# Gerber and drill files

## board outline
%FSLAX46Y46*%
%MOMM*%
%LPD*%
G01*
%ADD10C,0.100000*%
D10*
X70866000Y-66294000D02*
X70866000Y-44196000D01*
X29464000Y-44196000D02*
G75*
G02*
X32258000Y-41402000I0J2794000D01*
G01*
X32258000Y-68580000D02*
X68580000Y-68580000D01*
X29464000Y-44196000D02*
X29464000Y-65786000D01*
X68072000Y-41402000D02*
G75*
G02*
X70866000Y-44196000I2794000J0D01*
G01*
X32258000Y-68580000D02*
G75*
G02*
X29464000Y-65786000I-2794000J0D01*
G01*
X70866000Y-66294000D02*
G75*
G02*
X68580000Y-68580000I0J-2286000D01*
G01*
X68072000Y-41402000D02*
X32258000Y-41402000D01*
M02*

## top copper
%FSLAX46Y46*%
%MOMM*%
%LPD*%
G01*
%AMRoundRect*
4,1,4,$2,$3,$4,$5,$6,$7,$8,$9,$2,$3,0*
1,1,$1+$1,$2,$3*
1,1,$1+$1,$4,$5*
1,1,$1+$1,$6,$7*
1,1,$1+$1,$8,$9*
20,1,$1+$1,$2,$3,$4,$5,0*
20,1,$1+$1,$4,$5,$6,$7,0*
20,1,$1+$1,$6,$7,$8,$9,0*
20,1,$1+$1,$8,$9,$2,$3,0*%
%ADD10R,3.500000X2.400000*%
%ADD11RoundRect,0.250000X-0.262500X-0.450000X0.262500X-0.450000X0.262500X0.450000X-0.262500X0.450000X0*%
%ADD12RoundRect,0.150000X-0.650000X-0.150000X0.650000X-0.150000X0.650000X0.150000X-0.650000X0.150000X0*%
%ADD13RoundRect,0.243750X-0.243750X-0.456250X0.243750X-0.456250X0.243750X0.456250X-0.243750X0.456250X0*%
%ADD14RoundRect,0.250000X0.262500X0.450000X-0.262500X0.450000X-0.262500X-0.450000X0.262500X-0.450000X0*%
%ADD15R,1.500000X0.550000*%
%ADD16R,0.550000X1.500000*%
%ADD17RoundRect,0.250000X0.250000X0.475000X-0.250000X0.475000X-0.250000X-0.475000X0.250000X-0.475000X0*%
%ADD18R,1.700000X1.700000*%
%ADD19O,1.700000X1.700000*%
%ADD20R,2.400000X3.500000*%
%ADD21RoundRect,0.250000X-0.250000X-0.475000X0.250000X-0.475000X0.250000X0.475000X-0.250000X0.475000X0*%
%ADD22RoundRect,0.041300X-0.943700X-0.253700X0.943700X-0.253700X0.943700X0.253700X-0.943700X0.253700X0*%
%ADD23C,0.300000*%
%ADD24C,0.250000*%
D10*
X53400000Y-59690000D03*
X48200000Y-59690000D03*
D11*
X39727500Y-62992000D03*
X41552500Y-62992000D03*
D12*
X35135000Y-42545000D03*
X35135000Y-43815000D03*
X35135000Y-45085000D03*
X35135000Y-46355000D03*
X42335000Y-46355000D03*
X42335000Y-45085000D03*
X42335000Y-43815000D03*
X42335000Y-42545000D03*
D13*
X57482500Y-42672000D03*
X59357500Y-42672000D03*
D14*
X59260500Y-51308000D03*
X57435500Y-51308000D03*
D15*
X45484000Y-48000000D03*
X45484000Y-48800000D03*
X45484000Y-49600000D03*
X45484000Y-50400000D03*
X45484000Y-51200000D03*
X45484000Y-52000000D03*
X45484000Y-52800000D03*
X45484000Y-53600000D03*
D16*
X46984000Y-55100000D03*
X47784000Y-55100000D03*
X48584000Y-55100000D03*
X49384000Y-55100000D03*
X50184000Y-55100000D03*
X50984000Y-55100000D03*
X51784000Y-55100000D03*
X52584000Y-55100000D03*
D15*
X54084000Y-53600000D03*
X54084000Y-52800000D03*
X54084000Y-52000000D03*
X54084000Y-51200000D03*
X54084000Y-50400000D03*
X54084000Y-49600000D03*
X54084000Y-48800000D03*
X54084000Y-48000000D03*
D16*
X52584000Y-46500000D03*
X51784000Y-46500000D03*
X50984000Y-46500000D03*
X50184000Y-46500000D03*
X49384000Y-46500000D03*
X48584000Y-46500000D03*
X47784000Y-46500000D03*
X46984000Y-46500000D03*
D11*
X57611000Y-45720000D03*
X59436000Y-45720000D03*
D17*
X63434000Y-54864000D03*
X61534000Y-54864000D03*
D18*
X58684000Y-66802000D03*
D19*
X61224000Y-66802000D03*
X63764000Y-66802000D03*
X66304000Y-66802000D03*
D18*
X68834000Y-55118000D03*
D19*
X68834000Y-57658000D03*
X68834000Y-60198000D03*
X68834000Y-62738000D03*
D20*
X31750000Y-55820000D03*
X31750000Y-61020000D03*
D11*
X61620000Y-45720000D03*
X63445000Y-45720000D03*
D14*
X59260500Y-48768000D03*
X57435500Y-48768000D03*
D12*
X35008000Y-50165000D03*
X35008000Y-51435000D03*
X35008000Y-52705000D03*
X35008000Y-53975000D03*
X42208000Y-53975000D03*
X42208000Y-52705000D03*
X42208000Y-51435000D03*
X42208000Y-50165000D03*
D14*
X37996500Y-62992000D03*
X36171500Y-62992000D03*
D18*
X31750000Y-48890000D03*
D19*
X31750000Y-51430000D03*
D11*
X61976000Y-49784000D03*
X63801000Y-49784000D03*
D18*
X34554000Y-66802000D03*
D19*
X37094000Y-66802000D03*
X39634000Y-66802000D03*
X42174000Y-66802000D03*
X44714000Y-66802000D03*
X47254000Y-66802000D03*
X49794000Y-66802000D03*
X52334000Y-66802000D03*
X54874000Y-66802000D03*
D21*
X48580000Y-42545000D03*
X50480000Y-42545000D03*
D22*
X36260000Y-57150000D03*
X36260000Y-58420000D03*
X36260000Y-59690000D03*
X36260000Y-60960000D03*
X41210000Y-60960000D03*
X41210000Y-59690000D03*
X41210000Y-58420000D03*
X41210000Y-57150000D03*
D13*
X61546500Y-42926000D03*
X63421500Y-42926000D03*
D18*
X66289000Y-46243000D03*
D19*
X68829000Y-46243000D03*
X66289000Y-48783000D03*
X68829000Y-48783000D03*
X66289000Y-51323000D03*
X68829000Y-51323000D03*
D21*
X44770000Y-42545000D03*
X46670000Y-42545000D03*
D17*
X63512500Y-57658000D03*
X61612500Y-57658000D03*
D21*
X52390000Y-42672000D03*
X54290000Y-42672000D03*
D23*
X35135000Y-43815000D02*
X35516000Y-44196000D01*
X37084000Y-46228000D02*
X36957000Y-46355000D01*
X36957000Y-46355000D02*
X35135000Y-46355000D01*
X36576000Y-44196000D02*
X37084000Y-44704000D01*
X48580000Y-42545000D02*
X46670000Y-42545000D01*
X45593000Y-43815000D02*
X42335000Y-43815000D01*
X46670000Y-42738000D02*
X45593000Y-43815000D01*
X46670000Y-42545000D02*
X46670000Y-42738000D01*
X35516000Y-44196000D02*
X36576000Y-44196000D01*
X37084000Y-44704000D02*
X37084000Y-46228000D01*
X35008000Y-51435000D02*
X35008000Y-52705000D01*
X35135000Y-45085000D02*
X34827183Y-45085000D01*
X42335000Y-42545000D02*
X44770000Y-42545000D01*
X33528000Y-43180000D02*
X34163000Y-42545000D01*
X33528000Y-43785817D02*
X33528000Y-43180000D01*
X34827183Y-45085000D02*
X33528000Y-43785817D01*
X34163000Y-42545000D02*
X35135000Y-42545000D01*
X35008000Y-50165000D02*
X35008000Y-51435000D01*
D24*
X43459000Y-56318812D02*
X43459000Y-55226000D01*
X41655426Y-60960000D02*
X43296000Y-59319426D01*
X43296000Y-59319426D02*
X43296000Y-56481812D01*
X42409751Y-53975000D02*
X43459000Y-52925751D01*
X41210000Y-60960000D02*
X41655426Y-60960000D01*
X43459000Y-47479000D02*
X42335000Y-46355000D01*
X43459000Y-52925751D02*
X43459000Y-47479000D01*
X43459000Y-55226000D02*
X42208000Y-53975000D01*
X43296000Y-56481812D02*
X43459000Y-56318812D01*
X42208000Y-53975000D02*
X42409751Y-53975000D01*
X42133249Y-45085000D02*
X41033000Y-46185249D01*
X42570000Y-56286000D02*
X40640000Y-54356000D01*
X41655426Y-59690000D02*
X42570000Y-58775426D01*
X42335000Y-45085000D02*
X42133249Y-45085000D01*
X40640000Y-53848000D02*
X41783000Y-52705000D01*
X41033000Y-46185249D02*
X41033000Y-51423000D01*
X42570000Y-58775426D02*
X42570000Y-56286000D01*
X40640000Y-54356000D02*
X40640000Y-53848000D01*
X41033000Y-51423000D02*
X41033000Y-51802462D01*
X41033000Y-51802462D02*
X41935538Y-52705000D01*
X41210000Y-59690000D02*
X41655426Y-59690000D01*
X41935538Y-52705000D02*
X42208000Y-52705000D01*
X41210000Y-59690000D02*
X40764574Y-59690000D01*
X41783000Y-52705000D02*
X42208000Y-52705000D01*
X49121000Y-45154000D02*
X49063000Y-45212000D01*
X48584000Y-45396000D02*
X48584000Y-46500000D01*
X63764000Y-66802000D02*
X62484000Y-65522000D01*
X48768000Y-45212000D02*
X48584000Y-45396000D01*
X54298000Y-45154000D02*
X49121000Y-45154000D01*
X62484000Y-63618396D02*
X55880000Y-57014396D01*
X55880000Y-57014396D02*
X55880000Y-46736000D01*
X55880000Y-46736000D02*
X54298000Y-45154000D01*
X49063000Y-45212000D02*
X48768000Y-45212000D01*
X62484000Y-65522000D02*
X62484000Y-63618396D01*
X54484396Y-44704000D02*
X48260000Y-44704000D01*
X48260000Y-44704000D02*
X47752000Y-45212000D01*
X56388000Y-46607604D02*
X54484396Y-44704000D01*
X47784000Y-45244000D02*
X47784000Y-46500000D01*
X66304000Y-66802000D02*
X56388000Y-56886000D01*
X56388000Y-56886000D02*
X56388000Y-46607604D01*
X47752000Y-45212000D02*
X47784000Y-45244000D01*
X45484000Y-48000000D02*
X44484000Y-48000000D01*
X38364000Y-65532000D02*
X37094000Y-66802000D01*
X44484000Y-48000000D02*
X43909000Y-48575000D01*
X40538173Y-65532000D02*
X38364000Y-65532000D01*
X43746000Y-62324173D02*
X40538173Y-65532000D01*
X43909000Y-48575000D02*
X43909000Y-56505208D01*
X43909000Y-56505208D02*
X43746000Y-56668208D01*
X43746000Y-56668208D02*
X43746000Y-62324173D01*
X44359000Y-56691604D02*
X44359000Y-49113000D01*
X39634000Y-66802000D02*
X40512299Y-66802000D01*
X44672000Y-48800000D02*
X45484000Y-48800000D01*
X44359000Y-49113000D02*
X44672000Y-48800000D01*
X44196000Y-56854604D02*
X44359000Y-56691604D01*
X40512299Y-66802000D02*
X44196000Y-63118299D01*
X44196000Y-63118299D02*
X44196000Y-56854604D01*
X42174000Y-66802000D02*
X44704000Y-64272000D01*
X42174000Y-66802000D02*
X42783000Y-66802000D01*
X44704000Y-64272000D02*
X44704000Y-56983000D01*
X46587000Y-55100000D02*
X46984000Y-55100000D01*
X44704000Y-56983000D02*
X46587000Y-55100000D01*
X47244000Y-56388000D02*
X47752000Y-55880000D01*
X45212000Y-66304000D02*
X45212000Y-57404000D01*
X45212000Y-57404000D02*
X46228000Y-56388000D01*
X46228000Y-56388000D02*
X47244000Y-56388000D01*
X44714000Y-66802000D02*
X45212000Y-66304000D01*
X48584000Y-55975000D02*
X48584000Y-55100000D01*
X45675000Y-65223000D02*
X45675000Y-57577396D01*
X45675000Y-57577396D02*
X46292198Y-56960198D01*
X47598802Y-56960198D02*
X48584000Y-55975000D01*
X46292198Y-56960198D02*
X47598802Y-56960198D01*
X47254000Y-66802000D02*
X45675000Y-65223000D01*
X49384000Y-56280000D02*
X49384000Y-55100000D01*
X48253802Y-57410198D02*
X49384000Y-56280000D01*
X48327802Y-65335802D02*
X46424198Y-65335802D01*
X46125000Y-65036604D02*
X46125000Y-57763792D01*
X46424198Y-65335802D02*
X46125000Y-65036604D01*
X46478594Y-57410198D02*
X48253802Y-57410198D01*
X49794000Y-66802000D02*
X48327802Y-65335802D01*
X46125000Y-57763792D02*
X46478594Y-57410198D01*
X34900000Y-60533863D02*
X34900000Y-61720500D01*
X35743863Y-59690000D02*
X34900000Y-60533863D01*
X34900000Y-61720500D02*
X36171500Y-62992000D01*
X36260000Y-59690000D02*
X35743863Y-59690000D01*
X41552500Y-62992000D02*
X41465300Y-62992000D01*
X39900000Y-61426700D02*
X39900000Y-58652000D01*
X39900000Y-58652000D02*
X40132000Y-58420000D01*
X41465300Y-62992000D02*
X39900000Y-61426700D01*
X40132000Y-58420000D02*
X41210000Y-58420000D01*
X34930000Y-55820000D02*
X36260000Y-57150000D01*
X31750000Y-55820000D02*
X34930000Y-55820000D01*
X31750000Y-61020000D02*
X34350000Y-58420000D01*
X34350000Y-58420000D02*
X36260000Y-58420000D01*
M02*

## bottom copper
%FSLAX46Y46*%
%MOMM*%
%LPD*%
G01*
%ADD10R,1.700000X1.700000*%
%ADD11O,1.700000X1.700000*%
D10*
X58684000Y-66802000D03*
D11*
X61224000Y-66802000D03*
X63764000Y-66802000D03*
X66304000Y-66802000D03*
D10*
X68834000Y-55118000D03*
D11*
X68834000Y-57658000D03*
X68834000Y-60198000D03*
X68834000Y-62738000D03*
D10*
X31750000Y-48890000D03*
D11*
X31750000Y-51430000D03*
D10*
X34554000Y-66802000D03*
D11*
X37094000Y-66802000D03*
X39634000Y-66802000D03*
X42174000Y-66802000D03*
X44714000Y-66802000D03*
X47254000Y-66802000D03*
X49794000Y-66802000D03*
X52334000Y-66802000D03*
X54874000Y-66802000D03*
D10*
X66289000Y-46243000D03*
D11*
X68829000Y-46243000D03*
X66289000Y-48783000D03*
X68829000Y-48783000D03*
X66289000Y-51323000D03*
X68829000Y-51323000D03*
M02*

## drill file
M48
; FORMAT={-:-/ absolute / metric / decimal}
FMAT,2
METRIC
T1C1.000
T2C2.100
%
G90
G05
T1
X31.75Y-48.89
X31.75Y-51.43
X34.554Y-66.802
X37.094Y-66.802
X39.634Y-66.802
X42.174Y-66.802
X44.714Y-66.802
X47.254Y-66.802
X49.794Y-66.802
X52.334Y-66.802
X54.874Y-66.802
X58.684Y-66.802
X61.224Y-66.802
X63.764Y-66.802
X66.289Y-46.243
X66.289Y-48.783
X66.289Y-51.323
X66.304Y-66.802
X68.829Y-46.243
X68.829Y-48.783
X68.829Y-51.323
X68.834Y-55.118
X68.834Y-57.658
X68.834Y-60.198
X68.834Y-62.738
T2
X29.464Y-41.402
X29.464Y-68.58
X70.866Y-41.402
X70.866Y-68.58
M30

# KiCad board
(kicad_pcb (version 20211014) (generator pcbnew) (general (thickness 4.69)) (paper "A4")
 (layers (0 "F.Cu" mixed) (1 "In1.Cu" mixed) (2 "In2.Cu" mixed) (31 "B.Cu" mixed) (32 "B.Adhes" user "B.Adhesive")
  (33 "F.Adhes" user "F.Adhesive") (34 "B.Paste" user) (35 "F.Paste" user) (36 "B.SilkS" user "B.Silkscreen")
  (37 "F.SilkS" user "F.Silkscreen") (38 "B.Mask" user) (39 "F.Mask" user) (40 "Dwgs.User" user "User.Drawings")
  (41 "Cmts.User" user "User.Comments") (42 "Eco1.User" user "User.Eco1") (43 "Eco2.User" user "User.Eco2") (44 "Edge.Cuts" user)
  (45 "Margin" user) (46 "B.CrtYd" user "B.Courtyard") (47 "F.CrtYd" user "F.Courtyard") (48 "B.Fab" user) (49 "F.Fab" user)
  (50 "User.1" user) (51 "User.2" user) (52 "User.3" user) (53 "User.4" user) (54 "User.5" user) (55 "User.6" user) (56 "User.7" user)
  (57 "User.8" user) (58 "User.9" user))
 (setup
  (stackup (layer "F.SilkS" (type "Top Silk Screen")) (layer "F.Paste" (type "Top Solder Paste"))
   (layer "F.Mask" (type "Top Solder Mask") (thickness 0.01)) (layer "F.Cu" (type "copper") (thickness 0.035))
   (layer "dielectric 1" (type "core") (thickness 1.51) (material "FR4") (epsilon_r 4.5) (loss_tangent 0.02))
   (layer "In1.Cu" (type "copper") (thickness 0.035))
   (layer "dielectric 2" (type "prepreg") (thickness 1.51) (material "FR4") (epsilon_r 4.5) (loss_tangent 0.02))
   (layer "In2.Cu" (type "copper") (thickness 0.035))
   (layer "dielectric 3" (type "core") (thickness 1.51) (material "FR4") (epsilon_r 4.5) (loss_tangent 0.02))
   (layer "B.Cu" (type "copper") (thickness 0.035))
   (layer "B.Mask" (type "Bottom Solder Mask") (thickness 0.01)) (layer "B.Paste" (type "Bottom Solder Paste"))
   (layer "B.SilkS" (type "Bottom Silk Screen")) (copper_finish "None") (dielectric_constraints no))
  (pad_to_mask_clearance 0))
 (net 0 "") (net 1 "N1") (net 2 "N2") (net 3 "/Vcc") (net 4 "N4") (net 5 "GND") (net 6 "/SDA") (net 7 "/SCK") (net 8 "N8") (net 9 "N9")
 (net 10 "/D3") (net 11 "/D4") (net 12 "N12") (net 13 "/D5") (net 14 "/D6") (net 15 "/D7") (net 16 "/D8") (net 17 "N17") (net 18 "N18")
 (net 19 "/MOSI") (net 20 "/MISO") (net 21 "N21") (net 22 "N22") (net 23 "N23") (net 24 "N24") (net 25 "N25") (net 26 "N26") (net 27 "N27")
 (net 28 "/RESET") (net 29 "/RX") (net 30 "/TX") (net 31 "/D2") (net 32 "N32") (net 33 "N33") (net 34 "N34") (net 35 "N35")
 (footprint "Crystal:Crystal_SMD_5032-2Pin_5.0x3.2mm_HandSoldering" (layer "F.Cu") (at 50.8 59.69 180)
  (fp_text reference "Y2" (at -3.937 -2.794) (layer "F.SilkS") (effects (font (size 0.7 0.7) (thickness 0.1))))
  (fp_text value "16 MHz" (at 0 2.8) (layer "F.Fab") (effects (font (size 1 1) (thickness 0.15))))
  (pad "1" smd rect (at -2.6 0 180) (size 3.5 2.4) (layers "F.Cu" "F.Paste" "F.Mask") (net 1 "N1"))
  (pad "2" smd rect (at 2.6 0 180) (size 3.5 2.4) (layers "F.Cu" "F.Paste" "F.Mask") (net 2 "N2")))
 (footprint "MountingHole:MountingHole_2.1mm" (layer "F.Cu") (at 29.464 68.58)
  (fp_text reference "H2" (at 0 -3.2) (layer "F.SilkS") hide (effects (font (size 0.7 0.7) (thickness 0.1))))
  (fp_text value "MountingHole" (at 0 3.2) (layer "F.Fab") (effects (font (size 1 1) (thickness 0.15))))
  (pad "" np_thru_hole circle (at 0 0) (size 2.1 2.1) (drill 2.1) (layers *.Cu *.Mask)))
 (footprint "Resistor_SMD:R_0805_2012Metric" (layer "F.Cu") (at 40.64 62.992)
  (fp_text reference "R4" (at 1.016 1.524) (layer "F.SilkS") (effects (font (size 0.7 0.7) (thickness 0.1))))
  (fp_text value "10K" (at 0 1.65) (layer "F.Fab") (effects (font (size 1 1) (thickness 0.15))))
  (pad "1" smd roundrect (at -0.9125 0) (size 1.025 1.4) (layers "F.Cu" "F.Paste" "F.Mask") (roundrect_rratio 0.243902) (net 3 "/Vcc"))
  (pad "2" smd roundrect (at 0.9125 0) (size 1.025 1.4) (layers "F.Cu" "F.Paste" "F.Mask") (roundrect_rratio 0.243902) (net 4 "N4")))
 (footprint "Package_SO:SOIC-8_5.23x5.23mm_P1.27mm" (layer "F.Cu") (at 38.735 44.45)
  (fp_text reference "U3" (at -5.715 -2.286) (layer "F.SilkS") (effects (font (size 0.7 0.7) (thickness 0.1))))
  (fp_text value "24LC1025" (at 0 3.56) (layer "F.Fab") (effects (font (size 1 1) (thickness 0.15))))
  (pad "1" smd roundrect (at -3.6 -1.905) (size 1.6 0.6) (layers "F.Cu" "F.Paste" "F.Mask") (roundrect_rratio 0.25) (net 3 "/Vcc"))
  (pad "2" smd roundrect (at -3.6 -0.635) (size 1.6 0.6) (layers "F.Cu" "F.Paste" "F.Mask") (roundrect_rratio 0.25) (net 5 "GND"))
  (pad "3" smd roundrect (at -3.6 0.635) (size 1.6 0.6) (layers "F.Cu" "F.Paste" "F.Mask") (roundrect_rratio 0.25) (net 3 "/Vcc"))
  (pad "4" smd roundrect (at -3.6 1.905) (size 1.6 0.6) (layers "F.Cu" "F.Paste" "F.Mask") (roundrect_rratio 0.25) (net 5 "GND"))
  (pad "5" smd roundrect (at 3.6 1.905) (size 1.6 0.6) (layers "F.Cu" "F.Paste" "F.Mask") (roundrect_rratio 0.25) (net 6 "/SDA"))
  (pad "6" smd roundrect (at 3.6 0.635) (size 1.6 0.6) (layers "F.Cu" "F.Paste" "F.Mask") (roundrect_rratio 0.25) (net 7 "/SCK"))
  (pad "7" smd roundrect (at 3.6 -0.635) (size 1.6 0.6) (layers "F.Cu" "F.Paste" "F.Mask") (roundrect_rratio 0.25) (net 5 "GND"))
  (pad "8" smd roundrect (at 3.6 -1.905) (size 1.6 0.6) (layers "F.Cu" "F.Paste" "F.Mask") (roundrect_rratio 0.25) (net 3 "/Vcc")))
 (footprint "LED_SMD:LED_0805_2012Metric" (layer "F.Cu") (at 58.42 42.672)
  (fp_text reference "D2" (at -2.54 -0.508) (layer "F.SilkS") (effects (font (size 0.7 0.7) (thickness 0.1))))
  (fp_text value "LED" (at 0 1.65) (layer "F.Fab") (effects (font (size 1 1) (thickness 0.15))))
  (pad "1" smd roundrect (at -0.9375 0) (size 0.975 1.4) (layers "F.Cu" "F.Paste" "F.Mask") (roundrect_rratio 0.25) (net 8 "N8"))
  (pad "2" smd roundrect (at 0.9375 0) (size 0.975 1.4) (layers "F.Cu" "F.Paste" "F.Mask") (roundrect_rratio 0.25) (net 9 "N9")))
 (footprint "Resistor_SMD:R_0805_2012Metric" (layer "F.Cu") (at 58.348 51.308 180)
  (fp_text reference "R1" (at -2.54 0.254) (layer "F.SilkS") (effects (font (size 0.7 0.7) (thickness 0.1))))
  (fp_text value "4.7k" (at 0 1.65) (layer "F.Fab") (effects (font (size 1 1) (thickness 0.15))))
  (pad "1" smd roundrect (at -0.9125 0 180) (size 1.025 1.4) (layers "F.Cu" "F.Paste" "F.Mask") (roundrect_rratio 0.243902) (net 3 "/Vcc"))
  (pad "2" smd roundrect (at 0.9125 0 180) (size 1.025 1.4) (layers "F.Cu" "F.Paste" "F.Mask") (roundrect_rratio 0.243902) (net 7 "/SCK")))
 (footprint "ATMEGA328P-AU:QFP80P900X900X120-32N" (layer "F.Cu") (at 49.784 50.8)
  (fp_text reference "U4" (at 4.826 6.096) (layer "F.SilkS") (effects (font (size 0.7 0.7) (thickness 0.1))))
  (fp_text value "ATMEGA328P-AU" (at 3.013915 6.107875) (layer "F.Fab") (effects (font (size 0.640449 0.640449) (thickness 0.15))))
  (pad "1" smd rect locked (at -4.3 -2.8) (size 1.5 0.55) (layers "F.Cu" "F.Paste" "F.Mask") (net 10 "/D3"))
  (pad "2" smd rect locked (at -4.3 -2) (size 1.5 0.55) (layers "F.Cu" "F.Paste" "F.Mask") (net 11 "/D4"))
  (pad "3" smd rect locked (at -4.3 -1.2) (size 1.5 0.55) (layers "F.Cu" "F.Paste" "F.Mask") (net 5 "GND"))
  (pad "4" smd rect locked (at -4.3 -0.4) (size 1.5 0.55) (layers "F.Cu" "F.Paste" "F.Mask") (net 9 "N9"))
  (pad "5" smd rect locked (at -4.3 0.4) (size 1.5 0.55) (layers "F.Cu" "F.Paste" "F.Mask") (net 5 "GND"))
  (pad "6" smd rect locked (at -4.3 1.2) (size 1.5 0.55) (layers "F.Cu" "F.Paste" "F.Mask") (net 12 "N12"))
  (pad "7" smd rect locked (at -4.3 2) (size 1.5 0.55) (layers "F.Cu" "F.Paste" "F.Mask") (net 2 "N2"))
  (pad "8" smd rect locked (at -4.3 2.8) (size 1.5 0.55) (layers "F.Cu" "F.Paste" "F.Mask") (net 1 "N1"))
  (pad "9" smd rect locked (at -2.8 4.3) (size 0.55 1.5) (layers "F.Cu" "F.Paste" "F.Mask") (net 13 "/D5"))
  (pad "10" smd rect locked (at -2 4.3) (size 0.55 1.5) (layers "F.Cu" "F.Paste" "F.Mask") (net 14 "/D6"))
  (pad "11" smd rect locked (at -1.2 4.3) (size 0.55 1.5) (layers "F.Cu" "F.Paste" "F.Mask") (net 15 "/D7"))
  (pad "12" smd rect locked (at -0.4 4.3) (size 0.55 1.5) (layers "F.Cu" "F.Paste" "F.Mask") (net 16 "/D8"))
  (pad "13" smd rect locked (at 0.4 4.3) (size 0.55 1.5) (layers "F.Cu" "F.Paste" "F.Mask") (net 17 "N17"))
  (pad "14" smd rect locked (at 1.2 4.3) (size 0.55 1.5) (layers "F.Cu" "F.Paste" "F.Mask") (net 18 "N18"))
  (pad "15" smd rect locked (at 2 4.3) (size 0.55 1.5) (layers "F.Cu" "F.Paste" "F.Mask") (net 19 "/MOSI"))
  (pad "16" smd rect locked (at 2.8 4.3) (size 0.55 1.5) (layers "F.Cu" "F.Paste" "F.Mask") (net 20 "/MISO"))
  (pad "17" smd rect locked (at 4.3 2.8) (size 1.5 0.55) (layers "F.Cu" "F.Paste" "F.Mask") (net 7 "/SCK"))
  (pad "18" smd rect locked (at 4.3 2) (size 1.5 0.55) (layers "F.Cu" "F.Paste" "F.Mask") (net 9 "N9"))
  (pad "19" smd rect locked (at 4.3 1.2) (size 1.5 0.55) (layers "F.Cu" "F.Paste" "F.Mask") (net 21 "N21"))
  (pad "20" smd rect locked (at 4.3 0.4) (size 1.5 0.55) (layers "F.Cu" "F.Paste" "F.Mask") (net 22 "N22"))
  (pad "21" smd rect locked (at 4.3 -0.4) (size 1.5 0.55) (layers "F.Cu" "F.Paste" "F.Mask") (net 5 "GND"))
  (pad "22" smd rect locked (at 4.3 -1.2) (size 1.5 0.55) (layers "F.Cu" "F.Paste" "F.Mask") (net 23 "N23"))
  (pad "23" smd rect locked (at 4.3 -2) (size 1.5 0.55) (layers "F.Cu" "F.Paste" "F.Mask") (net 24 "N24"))
  (pad "24" smd rect locked (at 4.3 -2.8) (size 1.5 0.55) (layers "F.Cu" "F.Paste" "F.Mask") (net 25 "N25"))
  (pad "25" smd rect locked (at 2.8 -4.3) (size 0.55 1.5) (layers "F.Cu" "F.Paste" "F.Mask") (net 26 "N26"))
  (pad "26" smd rect locked (at 2 -4.3) (size 0.55 1.5) (layers "F.Cu" "F.Paste" "F.Mask") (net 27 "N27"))
  (pad "27" smd rect locked (at 1.2 -4.3) (size 0.55 1.5) (layers "F.Cu" "F.Paste" "F.Mask") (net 6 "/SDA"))
  (pad "28" smd rect locked (at 0.4 -4.3) (size 0.55 1.5) (layers "F.Cu" "F.Paste" "F.Mask") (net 7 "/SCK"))
  (pad "29" smd rect locked (at -0.4 -4.3) (size 0.55 1.5) (layers "F.Cu" "F.Paste" "F.Mask") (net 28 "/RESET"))
  (pad "30" smd rect locked (at -1.2 -4.3) (size 0.55 1.5) (layers "F.Cu" "F.Paste" "F.Mask") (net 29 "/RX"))
  (pad "31" smd rect locked (at -2 -4.3) (size 0.55 1.5) (layers "F.Cu" "F.Paste" "F.Mask") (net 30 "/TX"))
  (pad "32" smd rect locked (at -2.8 -4.3) (size 0.55 1.5) (layers "F.Cu" "F.Paste" "F.Mask") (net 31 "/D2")))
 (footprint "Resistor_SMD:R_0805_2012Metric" (layer "F.Cu") (at 58.5235 45.72)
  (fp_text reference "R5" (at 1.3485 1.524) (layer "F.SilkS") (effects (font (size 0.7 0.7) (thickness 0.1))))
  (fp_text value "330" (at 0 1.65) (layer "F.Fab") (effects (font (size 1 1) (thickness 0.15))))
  (pad "1" smd roundrect (at -0.9125 0) (size 1.025 1.4) (layers "F.Cu" "F.Paste" "F.Mask") (roundrect_rratio 0.243902) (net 5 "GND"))
  (pad "2" smd roundrect (at 0.9125 0) (size 1.025 1.4) (layers "F.Cu" "F.Paste" "F.Mask") (roundrect_rratio 0.243902) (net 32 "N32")))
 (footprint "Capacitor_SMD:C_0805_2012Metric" (layer "F.Cu") (at 62.484 54.864 180)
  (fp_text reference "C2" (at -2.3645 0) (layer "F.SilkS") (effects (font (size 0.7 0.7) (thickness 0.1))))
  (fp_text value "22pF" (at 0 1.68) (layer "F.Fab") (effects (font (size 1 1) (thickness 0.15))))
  (pad "1" smd roundrect (at -0.95 0 180) (size 1 1.45) (layers "F.Cu" "F.Paste" "F.Mask") (roundrect_rratio 0.25) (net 5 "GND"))
  (pad "2" smd roundrect (at 0.95 0 180) (size 1 1.45) (layers "F.Cu" "F.Paste" "F.Mask") (roundrect_rratio 0.25) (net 2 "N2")))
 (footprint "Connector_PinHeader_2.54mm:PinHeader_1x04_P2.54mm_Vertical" (layer "F.Cu") (at 58.684 66.802 90)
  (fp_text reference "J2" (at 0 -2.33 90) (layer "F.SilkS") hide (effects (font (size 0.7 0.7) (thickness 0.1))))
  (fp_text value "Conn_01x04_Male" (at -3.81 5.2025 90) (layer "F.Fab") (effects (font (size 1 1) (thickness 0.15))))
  (pad "1" thru_hole rect (at 0 0 90) (size 1.7 1.7) (drill 1) (layers *.Cu *.Mask) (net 5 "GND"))
  (pad "2" thru_hole oval (at 0 2.54 90) (size 1.7 1.7) (drill 1) (layers *.Cu *.Mask) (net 3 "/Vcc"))
  (pad "3" thru_hole oval (at 0 5.08 90) (size 1.7 1.7) (drill 1) (layers *.Cu *.Mask) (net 29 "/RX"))
  (pad "4" thru_hole oval (at 0 7.62 90) (size 1.7 1.7) (drill 1) (layers *.Cu *.Mask) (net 30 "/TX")))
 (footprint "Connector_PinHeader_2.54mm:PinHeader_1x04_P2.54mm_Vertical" (layer "F.Cu") (at 68.834 55.118)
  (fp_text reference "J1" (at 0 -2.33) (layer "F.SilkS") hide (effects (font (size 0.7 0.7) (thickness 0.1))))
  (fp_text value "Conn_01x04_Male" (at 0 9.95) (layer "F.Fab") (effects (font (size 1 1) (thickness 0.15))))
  (pad "1" thru_hole rect (at 0 0) (size 1.7 1.7) (drill 1) (layers *.Cu *.Mask) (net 5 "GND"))
  (pad "2" thru_hole oval (at 0 2.54) (size 1.7 1.7) (drill 1) (layers *.Cu *.Mask) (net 3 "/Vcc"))
  (pad "3" thru_hole oval (at 0 5.08) (size 1.7 1.7) (drill 1) (layers *.Cu *.Mask) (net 6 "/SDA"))
  (pad "4" thru_hole oval (at 0 7.62) (size 1.7 1.7) (drill 1) (layers *.Cu *.Mask) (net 7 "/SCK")))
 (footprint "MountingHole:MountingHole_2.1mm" (layer "F.Cu") (at 70.866 68.58)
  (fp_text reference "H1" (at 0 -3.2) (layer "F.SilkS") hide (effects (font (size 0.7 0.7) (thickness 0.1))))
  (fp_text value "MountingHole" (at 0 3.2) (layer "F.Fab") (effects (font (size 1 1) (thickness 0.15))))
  (pad "" np_thru_hole circle (at 0 0) (size 2.1 2.1) (drill 2.1) (layers *.Cu *.Mask)))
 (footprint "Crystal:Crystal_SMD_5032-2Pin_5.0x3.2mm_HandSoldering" (layer "F.Cu") (at 31.75 58.42 -90)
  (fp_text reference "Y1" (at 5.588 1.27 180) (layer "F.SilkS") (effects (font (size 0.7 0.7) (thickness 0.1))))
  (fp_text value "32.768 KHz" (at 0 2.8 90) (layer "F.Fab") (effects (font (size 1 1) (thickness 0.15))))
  (pad "1" smd rect (at -2.6 0 270) (size 3.5 2.4) (layers "F.Cu" "F.Paste" "F.Mask") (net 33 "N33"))
  (pad "2" smd rect (at 2.6 0 270) (size 3.5 2.4) (layers "F.Cu" "F.Paste" "F.Mask") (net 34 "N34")))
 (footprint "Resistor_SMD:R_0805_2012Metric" (layer "F.Cu") (at 62.5325 45.72)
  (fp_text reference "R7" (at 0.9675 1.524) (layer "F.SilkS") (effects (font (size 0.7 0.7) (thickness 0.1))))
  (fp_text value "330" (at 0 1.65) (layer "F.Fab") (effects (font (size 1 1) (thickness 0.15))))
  (pad "1" smd roundrect (at -0.9125 0) (size 1.025 1.4) (layers "F.Cu" "F.Paste" "F.Mask") (roundrect_rratio 0.243902) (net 8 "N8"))
  (pad "2" smd roundrect (at 0.9125 0) (size 1.025 1.4) (layers "F.Cu" "F.Paste" "F.Mask") (roundrect_rratio 0.243902) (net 5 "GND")))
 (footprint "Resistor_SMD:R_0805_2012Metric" (layer "F.Cu") (at 58.348 48.768 180)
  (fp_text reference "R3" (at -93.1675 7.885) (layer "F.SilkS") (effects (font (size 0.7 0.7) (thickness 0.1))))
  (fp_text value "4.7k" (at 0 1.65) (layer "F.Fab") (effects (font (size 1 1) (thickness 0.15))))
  (pad "1" smd roundrect (at -0.9125 0 180) (size 1.025 1.4) (layers "F.Cu" "F.Paste" "F.Mask") (roundrect_rratio 0.243902) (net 3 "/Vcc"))
  (pad "2" smd roundrect (at 0.9125 0 180) (size 1.025 1.4) (layers "F.Cu" "F.Paste" "F.Mask") (roundrect_rratio 0.243902) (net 6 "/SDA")))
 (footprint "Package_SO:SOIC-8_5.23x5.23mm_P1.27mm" (layer "F.Cu") (at 38.608 52.07)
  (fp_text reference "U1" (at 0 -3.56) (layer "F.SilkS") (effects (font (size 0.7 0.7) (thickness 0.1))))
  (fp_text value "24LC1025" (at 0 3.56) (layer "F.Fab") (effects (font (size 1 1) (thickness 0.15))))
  (pad "1" smd roundrect (at -3.6 -1.905) (size 1.6 0.6) (layers "F.Cu" "F.Paste" "F.Mask") (roundrect_rratio 0.25) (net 3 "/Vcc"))
  (pad "2" smd roundrect (at -3.6 -0.635) (size 1.6 0.6) (layers "F.Cu" "F.Paste" "F.Mask") (roundrect_rratio 0.25) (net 3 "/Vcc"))
  (pad "3" smd roundrect (at -3.6 0.635) (size 1.6 0.6) (layers "F.Cu" "F.Paste" "F.Mask") (roundrect_rratio 0.25) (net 3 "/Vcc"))
  (pad "4" smd roundrect (at -3.6 1.905) (size 1.6 0.6) (layers "F.Cu" "F.Paste" "F.Mask") (roundrect_rratio 0.25) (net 5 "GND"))
  (pad "5" smd roundrect (at 3.6 1.905) (size 1.6 0.6) (layers "F.Cu" "F.Paste" "F.Mask") (roundrect_rratio 0.25) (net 6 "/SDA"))
  (pad "6" smd roundrect (at 3.6 0.635) (size 1.6 0.6) (layers "F.Cu" "F.Paste" "F.Mask") (roundrect_rratio 0.25) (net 7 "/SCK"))
  (pad "7" smd roundrect (at 3.6 -0.635) (size 1.6 0.6) (layers "F.Cu" "F.Paste" "F.Mask") (roundrect_rratio 0.25) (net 5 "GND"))
  (pad "8" smd roundrect (at 3.6 -1.905) (size 1.6 0.6) (layers "F.Cu" "F.Paste" "F.Mask") (roundrect_rratio 0.25) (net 3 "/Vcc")))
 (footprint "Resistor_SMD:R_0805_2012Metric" (layer "F.Cu") (at 37.084 62.992 180)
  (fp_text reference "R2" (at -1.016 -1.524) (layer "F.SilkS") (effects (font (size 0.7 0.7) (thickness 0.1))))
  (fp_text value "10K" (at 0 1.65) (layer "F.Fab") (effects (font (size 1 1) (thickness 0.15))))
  (pad "1" smd roundrect (at -0.9125 0 180) (size 1.025 1.4) (layers "F.Cu" "F.Paste" "F.Mask") (roundrect_rratio 0.243902) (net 3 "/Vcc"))
  (pad "2" smd roundrect (at 0.9125 0 180) (size 1.025 1.4) (layers "F.Cu" "F.Paste" "F.Mask") (roundrect_rratio 0.243902) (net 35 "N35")))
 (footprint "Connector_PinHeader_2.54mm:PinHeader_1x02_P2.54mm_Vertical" (layer "F.Cu") (at 31.75 48.89)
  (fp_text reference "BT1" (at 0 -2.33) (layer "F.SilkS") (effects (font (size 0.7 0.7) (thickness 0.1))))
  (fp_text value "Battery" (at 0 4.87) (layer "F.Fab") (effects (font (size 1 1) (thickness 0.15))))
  (pad "1" thru_hole rect (at 0 0) (size 1.7 1.7) (drill 1) (layers *.Cu *.Mask) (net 9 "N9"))
  (pad "2" thru_hole oval (at 0 2.54) (size 1.7 1.7) (drill 1) (layers *.Cu *.Mask) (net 5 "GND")))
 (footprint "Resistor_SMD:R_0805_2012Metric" (layer "F.Cu") (at 62.8885 49.784)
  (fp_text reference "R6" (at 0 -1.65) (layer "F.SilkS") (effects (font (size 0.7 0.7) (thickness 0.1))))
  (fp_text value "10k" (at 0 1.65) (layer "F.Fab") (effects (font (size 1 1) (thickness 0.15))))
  (pad "1" smd roundrect (at -0.9125 0) (size 1.025 1.4) (layers "F.Cu" "F.Paste" "F.Mask") (roundrect_rratio 0.243902) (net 3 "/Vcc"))
  (pad "2" smd roundrect (at 0.9125 0) (size 1.025 1.4) (layers "F.Cu" "F.Paste" "F.Mask") (roundrect_rratio 0.243902) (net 28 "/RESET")))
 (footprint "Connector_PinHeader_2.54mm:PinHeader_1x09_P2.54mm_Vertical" (layer "F.Cu") (at 34.554 66.802 90)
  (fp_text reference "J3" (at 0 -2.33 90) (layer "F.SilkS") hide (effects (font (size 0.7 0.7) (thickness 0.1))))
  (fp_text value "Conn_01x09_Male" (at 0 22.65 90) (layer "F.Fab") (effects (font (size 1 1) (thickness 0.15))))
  (pad "1" thru_hole rect (at 0 0 90) (size 1.7 1.7) (drill 1) (layers *.Cu *.Mask) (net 31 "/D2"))
  (pad "2" thru_hole oval (at 0 2.54 90) (size 1.7 1.7) (drill 1) (layers *.Cu *.Mask) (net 10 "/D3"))
  (pad "3" thru_hole oval (at 0 5.08 90) (size 1.7 1.7) (drill 1) (layers *.Cu *.Mask) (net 11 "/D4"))
  (pad "4" thru_hole oval (at 0 7.62 90) (size 1.7 1.7) (drill 1) (layers *.Cu *.Mask) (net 13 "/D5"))
  (pad "5" thru_hole oval (at 0 10.16 90) (size 1.7 1.7) (drill 1) (layers *.Cu *.Mask) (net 14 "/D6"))
  (pad "6" thru_hole oval (at 0 12.7 90) (size 1.7 1.7) (drill 1) (layers *.Cu *.Mask) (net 15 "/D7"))
  (pad "7" thru_hole oval (at 0 15.24 90) (size 1.7 1.7) (drill 1) (layers *.Cu *.Mask) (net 16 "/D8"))
  (pad "8" thru_hole oval (at 0 17.78 90) (size 1.7 1.7) (drill 1) (layers *.Cu *.Mask) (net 5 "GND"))
  (pad "9" thru_hole oval (at 0 20.32 90) (size 1.7 1.7) (drill 1) (layers *.Cu *.Mask) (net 3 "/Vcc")))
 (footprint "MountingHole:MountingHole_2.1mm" (layer "F.Cu") (at 29.464 41.402)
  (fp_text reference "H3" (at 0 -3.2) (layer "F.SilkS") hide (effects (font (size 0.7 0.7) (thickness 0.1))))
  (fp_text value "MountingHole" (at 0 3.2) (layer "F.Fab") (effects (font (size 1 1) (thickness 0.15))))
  (pad "" np_thru_hole circle (at 0 0) (size 2.1 2.1) (drill 2.1) (layers *.Cu *.Mask)))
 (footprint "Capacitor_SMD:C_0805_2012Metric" (layer "F.Cu") (at 49.53 42.545)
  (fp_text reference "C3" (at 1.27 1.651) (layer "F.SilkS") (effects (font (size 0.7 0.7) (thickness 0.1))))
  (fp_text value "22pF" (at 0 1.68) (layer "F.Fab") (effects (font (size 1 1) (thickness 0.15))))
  (pad "1" smd roundrect (at -0.95 0) (size 1 1.45) (layers "F.Cu" "F.Paste" "F.Mask") (roundrect_rratio 0.25) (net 5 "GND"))
  (pad "2" smd roundrect (at 0.95 0) (size 1 1.45) (layers "F.Cu" "F.Paste" "F.Mask") (roundrect_rratio 0.25) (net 1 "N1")))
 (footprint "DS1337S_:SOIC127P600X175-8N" (layer "F.Cu") (at 38.735 59.055)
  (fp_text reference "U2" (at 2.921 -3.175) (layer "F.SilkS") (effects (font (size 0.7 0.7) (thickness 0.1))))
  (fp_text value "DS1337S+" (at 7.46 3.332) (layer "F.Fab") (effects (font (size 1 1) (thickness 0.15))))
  (pad "1" smd roundrect locked (at -2.475 -1.905) (size 1.97 0.59) (layers "F.Cu" "F.Paste" "F.Mask") (roundrect_rratio 0.07)
   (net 33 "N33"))
  (pad "2" smd roundrect locked (at -2.475 -0.635) (size 1.97 0.59) (layers "F.Cu" "F.Paste" "F.Mask") (roundrect_rratio 0.07)
   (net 34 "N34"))
  (pad "3" smd roundrect locked (at -2.475 0.635) (size 1.97 0.59) (layers "F.Cu" "F.Paste" "F.Mask") (roundrect_rratio 0.07) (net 35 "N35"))
  (pad "4" smd roundrect locked (at -2.475 1.905) (size 1.97 0.59) (layers "F.Cu" "F.Paste" "F.Mask") (roundrect_rratio 0.07) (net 5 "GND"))
  (pad "5" smd roundrect locked (at 2.475 1.905) (size 1.97 0.59) (layers "F.Cu" "F.Paste" "F.Mask") (roundrect_rratio 0.07) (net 6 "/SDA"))
  (pad "6" smd roundrect locked (at 2.475 0.635) (size 1.97 0.59) (layers "F.Cu" "F.Paste" "F.Mask") (roundrect_rratio 0.07) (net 7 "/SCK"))
  (pad "7" smd roundrect locked (at 2.475 -0.635) (size 1.97 0.59) (layers "F.Cu" "F.Paste" "F.Mask") (roundrect_rratio 0.07) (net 4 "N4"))
  (pad "8" smd roundrect locked (at 2.475 -1.905) (size 1.97 0.59) (layers "F.Cu" "F.Paste" "F.Mask") (roundrect_rratio 0.07) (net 3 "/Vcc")))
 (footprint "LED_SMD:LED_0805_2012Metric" (layer "F.Cu") (at 62.484 42.926)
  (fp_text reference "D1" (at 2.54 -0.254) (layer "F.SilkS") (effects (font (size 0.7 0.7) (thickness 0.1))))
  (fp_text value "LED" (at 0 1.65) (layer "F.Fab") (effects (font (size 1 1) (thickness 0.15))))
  (pad "1" smd roundrect (at -0.9375 0) (size 0.975 1.4) (layers "F.Cu" "F.Paste" "F.Mask") (roundrect_rratio 0.25) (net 32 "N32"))
  (pad "2" smd roundrect (at 0.9375 0) (size 0.975 1.4) (layers "F.Cu" "F.Paste" "F.Mask") (roundrect_rratio 0.25) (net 7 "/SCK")))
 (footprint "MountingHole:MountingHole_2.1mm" (layer "F.Cu") (at 70.866 41.402)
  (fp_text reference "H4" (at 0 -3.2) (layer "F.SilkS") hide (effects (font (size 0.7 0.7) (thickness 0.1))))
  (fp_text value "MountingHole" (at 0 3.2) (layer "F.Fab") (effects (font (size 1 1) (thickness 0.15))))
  (pad "" np_thru_hole circle (at 0 0) (size 2.1 2.1) (drill 2.1) (layers *.Cu *.Mask)))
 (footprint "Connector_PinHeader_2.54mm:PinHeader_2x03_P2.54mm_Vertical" (layer "F.Cu") (at 66.289 46.243)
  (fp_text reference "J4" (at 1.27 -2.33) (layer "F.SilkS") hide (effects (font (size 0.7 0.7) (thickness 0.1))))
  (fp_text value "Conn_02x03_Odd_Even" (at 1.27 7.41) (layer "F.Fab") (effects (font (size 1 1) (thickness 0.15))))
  (pad "1" thru_hole rect (at 0 0) (size 1.7 1.7) (drill 1) (layers *.Cu *.Mask) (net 20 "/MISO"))
  (pad "2" thru_hole oval (at 2.54 0) (size 1.7 1.7) (drill 1) (layers *.Cu *.Mask) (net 3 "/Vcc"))
  (pad "3" thru_hole oval (at 0 2.54) (size 1.7 1.7) (drill 1) (layers *.Cu *.Mask) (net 7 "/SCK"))
  (pad "4" thru_hole oval (at 2.54 2.54) (size 1.7 1.7) (drill 1) (layers *.Cu *.Mask) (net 19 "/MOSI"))
  (pad "5" thru_hole oval (at 0 5.08) (size 1.7 1.7) (drill 1) (layers *.Cu *.Mask) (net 28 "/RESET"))
  (pad "6" thru_hole oval (at 2.54 5.08) (size 1.7 1.7) (drill 1) (layers *.Cu *.Mask) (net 5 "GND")))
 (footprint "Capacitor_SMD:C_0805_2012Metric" (layer "F.Cu") (at 45.72 42.545)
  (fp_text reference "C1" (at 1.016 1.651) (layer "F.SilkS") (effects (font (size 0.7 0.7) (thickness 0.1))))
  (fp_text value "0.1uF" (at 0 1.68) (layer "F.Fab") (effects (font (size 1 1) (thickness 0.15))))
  (pad "1" smd roundrect (at -0.95 0) (size 1 1.45) (layers "F.Cu" "F.Paste" "F.Mask") (roundrect_rratio 0.25) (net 3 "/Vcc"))
  (pad "2" smd roundrect (at 0.95 0) (size 1 1.45) (layers "F.Cu" "F.Paste" "F.Mask") (roundrect_rratio 0.25) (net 5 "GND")))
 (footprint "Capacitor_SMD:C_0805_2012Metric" (layer "F.Cu") (at 62.5625 57.658 180)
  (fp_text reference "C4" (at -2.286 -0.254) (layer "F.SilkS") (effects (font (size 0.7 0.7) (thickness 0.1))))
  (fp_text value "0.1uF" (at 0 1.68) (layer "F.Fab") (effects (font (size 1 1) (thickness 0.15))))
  (pad "1" smd roundrect (at -0.95 0 180) (size 1 1.45) (layers "F.Cu" "F.Paste" "F.Mask") (roundrect_rratio 0.25) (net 5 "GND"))
  (pad "2" smd roundrect (at 0.95 0 180) (size 1 1.45) (layers "F.Cu" "F.Paste" "F.Mask") (roundrect_rratio 0.25) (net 22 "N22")))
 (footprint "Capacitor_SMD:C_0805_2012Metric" (layer "F.Cu") (at 53.34 42.672)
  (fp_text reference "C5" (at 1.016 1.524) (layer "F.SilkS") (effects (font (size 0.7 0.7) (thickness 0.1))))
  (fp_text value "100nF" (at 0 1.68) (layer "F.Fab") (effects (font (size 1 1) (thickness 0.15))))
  (pad "1" smd roundrect (at -0.95 0) (size 1 1.45) (layers "F.Cu" "F.Paste" "F.Mask") (roundrect_rratio 0.25) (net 9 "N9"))
  (pad "2" smd roundrect (at 0.95 0) (size 1 1.45) (layers "F.Cu" "F.Paste" "F.Mask") (roundrect_rratio 0.25) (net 5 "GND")))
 (gr_line (start 70.866 66.294) (end 70.866 44.196) (layer "Edge.Cuts") (width 0.1))
 (gr_arc (start 29.464 44.196) (mid 27.488344 39.426344) (end 32.258 41.402) (layer "Edge.Cuts") (width 0.1))
 (gr_line (start 32.258 68.58) (end 68.58 68.58) (layer "Edge.Cuts") (width 0.1))
 (gr_line (start 29.464 44.196) (end 29.464 65.786) (layer "Edge.Cuts") (width 0.1))
 (gr_arc (start 68.072 41.402) (mid 72.841656 39.426344) (end 70.866 44.196) (layer "Edge.Cuts") (width 0.1))
 (gr_arc (start 32.258 68.58) (mid 27.488344 70.555656) (end 29.464 65.786) (layer "Edge.Cuts") (width 0.1))
 (gr_arc (start 70.866 66.294) (mid 72.482446 70.196446) (end 68.58 68.58) (layer "Edge.Cuts") (width 0.1))
 (gr_line (start 68.072 41.402) (end 32.258 41.402) (layer "Edge.Cuts") (width 0.1))
 (segment (start 35.135 43.815) (end 35.516 44.196) (width 0.3) (layer "F.Cu") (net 5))
 (segment (start 37.084 46.228) (end 36.957 46.355) (width 0.3) (layer "F.Cu") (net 5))
 (segment (start 36.957 46.355) (end 35.135 46.355) (width 0.3) (layer "F.Cu") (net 5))
 (segment (start 36.576 44.196) (end 37.084 44.704) (width 0.3) (layer "F.Cu") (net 5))
 (segment (start 48.58 42.545) (end 46.67 42.545) (width 0.3) (layer "F.Cu") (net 5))
 (segment (start 45.593 43.815) (end 42.335 43.815) (width 0.3) (layer "F.Cu") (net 5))
 (segment (start 46.67 42.738) (end 45.593 43.815) (width 0.3) (layer "F.Cu") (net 5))
 (segment (start 46.67 42.545) (end 46.67 42.738) (width 0.3) (layer "F.Cu") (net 5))
 (segment (start 35.516 44.196) (end 36.576 44.196) (width 0.3) (layer "F.Cu") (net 5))
 (segment (start 37.084 44.704) (end 37.084 46.228) (width 0.3) (layer "F.Cu") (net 5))
 (segment (start 35.008 51.435) (end 35.008 52.705) (width 0.3) (layer "F.Cu") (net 3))
 (segment (start 35.135 45.085) (end 34.827183 45.085) (width 0.3) (layer "F.Cu") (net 3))
 (segment (start 42.335 42.545) (end 44.77 42.545) (width 0.3) (layer "F.Cu") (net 3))
 (segment (start 33.528 43.18) (end 34.163 42.545) (width 0.3) (layer "F.Cu") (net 3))
 (segment (start 33.528 43.785817) (end 33.528 43.18) (width 0.3) (layer "F.Cu") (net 3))
 (segment (start 34.827183 45.085) (end 33.528 43.785817) (width 0.3) (layer "F.Cu") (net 3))
 (segment (start 34.163 42.545) (end 35.135 42.545) (width 0.3) (layer "F.Cu") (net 3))
 (segment (start 35.008 50.165) (end 35.008 51.435) (width 0.3) (layer "F.Cu") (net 3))
 (segment (start 43.459 56.318812) (end 43.459 55.226) (width 0.25) (layer "F.Cu") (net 6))
 (segment (start 41.655426 60.96) (end 43.296 59.319426) (width 0.25) (layer "F.Cu") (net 6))
 (segment (start 43.296 59.319426) (end 43.296 56.481812) (width 0.25) (layer "F.Cu") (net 6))
 (segment (start 42.409751 53.975) (end 43.459 52.925751) (width 0.25) (layer "F.Cu") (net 6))
 (segment (start 41.21 60.96) (end 41.655426 60.96) (width 0.25) (layer "F.Cu") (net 6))
 (segment (start 43.459 47.479) (end 42.335 46.355) (width 0.25) (layer "F.Cu") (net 6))
 (segment (start 43.459 52.925751) (end 43.459 47.479) (width 0.25) (layer "F.Cu") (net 6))
 (segment (start 43.459 55.226) (end 42.208 53.975) (width 0.25) (layer "F.Cu") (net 6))
 (segment (start 43.296 56.481812) (end 43.459 56.318812) (width 0.25) (layer "F.Cu") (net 6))
 (segment (start 42.208 53.975) (end 42.409751 53.975) (width 0.25) (layer "F.Cu") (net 6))
 (segment (start 42.133249 45.085) (end 41.033 46.185249) (width 0.25) (layer "F.Cu") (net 7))
 (segment (start 42.57 56.286) (end 40.64 54.356) (width 0.25) (layer "F.Cu") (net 7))
 (segment (start 41.655426 59.69) (end 42.57 58.775426) (width 0.25) (layer "F.Cu") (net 7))
 (segment (start 42.335 45.085) (end 42.133249 45.085) (width 0.25) (layer "F.Cu") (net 7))
 (segment (start 40.64 53.848) (end 41.783 52.705) (width 0.25) (layer "F.Cu") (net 7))
 (segment (start 41.033 46.185249) (end 41.033 51.423) (width 0.25) (layer "F.Cu") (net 7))
 (segment (start 42.57 58.775426) (end 42.57 56.286) (width 0.25) (layer "F.Cu") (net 7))
 (segment (start 40.64 54.356) (end 40.64 53.848) (width 0.25) (layer "F.Cu") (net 7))
 (segment (start 41.033 51.423) (end 41.033 51.802462) (width 0.25) (layer "F.Cu") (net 7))
 (segment (start 41.033 51.802462) (end 41.935538 52.705) (width 0.25) (layer "F.Cu") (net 7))
 (segment (start 41.21 59.69) (end 41.655426 59.69) (width 0.25) (layer "F.Cu") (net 7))
 (segment (start 41.935538 52.705) (end 42.208 52.705) (width 0.25) (layer "F.Cu") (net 7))
 (segment (start 41.21 59.69) (end 40.764574 59.69) (width 0.25) (layer "F.Cu") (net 7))
 (segment (start 41.783 52.705) (end 42.208 52.705) (width 0.25) (layer "F.Cu") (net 7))
 (segment (start 49.121 45.154) (end 49.063 45.212) (width 0.25) (layer "F.Cu") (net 29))
 (segment (start 48.584 45.396) (end 48.584 46.5) (width 0.25) (layer "F.Cu") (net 29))
 (segment (start 63.764 66.802) (end 62.484 65.522) (width 0.25) (layer "F.Cu") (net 29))
 (segment (start 48.768 45.212) (end 48.584 45.396) (width 0.25) (layer "F.Cu") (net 29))
 (segment (start 54.298 45.154) (end 49.121 45.154) (width 0.25) (layer "F.Cu") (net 29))
 (segment (start 62.484 63.618396) (end 55.88 57.014396) (width 0.25) (layer "F.Cu") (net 29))
 (segment (start 55.88 57.014396) (end 55.88 46.736) (width 0.25) (layer "F.Cu") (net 29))
 (segment (start 55.88 46.736) (end 54.298 45.154) (width 0.25) (layer "F.Cu") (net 29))
 (segment (start 49.063 45.212) (end 48.768 45.212) (width 0.25) (layer "F.Cu") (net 29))
 (segment (start 62.484 65.522) (end 62.484 63.618396) (width 0.25) (layer "F.Cu") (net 29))
 (segment (start 54.484396 44.704) (end 48.26 44.704) (width 0.25) (layer "F.Cu") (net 30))
 (segment (start 48.26 44.704) (end 47.752 45.212) (width 0.25) (layer "F.Cu") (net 30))
 (segment (start 56.388 46.607604) (end 54.484396 44.704) (width 0.25) (layer "F.Cu") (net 30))
 (segment (start 47.784 45.244) (end 47.784 46.5) (width 0.25) (layer "F.Cu") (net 30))
 (segment (start 66.304 66.802) (end 56.388 56.886) (width 0.25) (layer "F.Cu") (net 30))
 (segment (start 56.388 56.886) (end 56.388 46.607604) (width 0.25) (layer "F.Cu") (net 30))
 (segment (start 47.752 45.212) (end 47.784 45.244) (width 0.25) (layer "F.Cu") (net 30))
 (segment (start 45.484 48) (end 44.484 48) (width 0.25) (layer "F.Cu") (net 10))
 (segment (start 38.364 65.532) (end 37.094 66.802) (width 0.25) (layer "F.Cu") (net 10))
 (segment (start 44.484 48) (end 43.909 48.575) (width 0.25) (layer "F.Cu") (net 10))
 (segment (start 40.538173 65.532) (end 38.364 65.532) (width 0.25) (layer "F.Cu") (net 10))
 (segment (start 43.746 62.324173) (end 40.538173 65.532) (width 0.25) (layer "F.Cu") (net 10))
 (segment (start 43.909 48.575) (end 43.909 56.505208) (width 0.25) (layer "F.Cu") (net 10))
 (segment (start 43.909 56.505208) (end 43.746 56.668208) (width 0.25) (layer "F.Cu") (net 10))
 (segment (start 43.746 56.668208) (end 43.746 62.324173) (width 0.25) (layer "F.Cu") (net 10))
 (segment (start 44.359 56.691604) (end 44.359 49.113) (width 0.25) (layer "F.Cu") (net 11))
 (segment (start 39.634 66.802) (end 40.512299 66.802) (width 0.25) (layer "F.Cu") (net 11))
 (segment (start 44.672 48.8) (end 45.484 48.8) (width 0.25) (layer "F.Cu") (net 11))
 (segment (start 44.359 49.113) (end 44.672 48.8) (width 0.25) (layer "F.Cu") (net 11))
 (segment (start 44.196 56.854604) (end 44.359 56.691604) (width 0.25) (layer "F.Cu") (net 11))
 (segment (start 40.512299 66.802) (end 44.196 63.118299) (width 0.25) (layer "F.Cu") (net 11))
 (segment (start 44.196 63.118299) (end 44.196 56.854604) (width 0.25) (layer "F.Cu") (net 11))
 (segment (start 42.174 66.802) (end 44.704 64.272) (width 0.25) (layer "F.Cu") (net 13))
 (segment (start 42.174 66.802) (end 42.783 66.802) (width 0.25) (layer "F.Cu") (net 13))
 (segment (start 44.704 64.272) (end 44.704 56.983) (width 0.25) (layer "F.Cu") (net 13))
 (segment (start 46.587 55.1) (end 46.984 55.1) (width 0.25) (layer "F.Cu") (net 13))
 (segment (start 44.704 56.983) (end 46.587 55.1) (width 0.25) (layer "F.Cu") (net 13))
 (segment (start 47.244 56.388) (end 47.752 55.88) (width 0.25) (layer "F.Cu") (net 14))
 (segment (start 45.212 66.304) (end 45.212 57.404) (width 0.25) (layer "F.Cu") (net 14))
 (segment (start 45.212 57.404) (end 46.228 56.388) (width 0.25) (layer "F.Cu") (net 14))
 (segment (start 46.228 56.388) (end 47.244 56.388) (width 0.25) (layer "F.Cu") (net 14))
 (segment (start 44.714 66.802) (end 45.212 66.304) (width 0.25) (layer "F.Cu") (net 14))
 (segment (start 48.584 55.975) (end 48.584 55.1) (width 0.25) (layer "F.Cu") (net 15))
 (segment (start 45.675 65.223) (end 45.675 57.577396) (width 0.25) (layer "F.Cu") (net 15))
 (segment (start 45.675 57.577396) (end 46.292198 56.960198) (width 0.25) (layer "F.Cu") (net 15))
 (segment (start 47.598802 56.960198) (end 48.584 55.975) (width 0.25) (layer "F.Cu") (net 15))
 (segment (start 46.292198 56.960198) (end 47.598802 56.960198) (width 0.25) (layer "F.Cu") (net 15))
 (segment (start 47.254 66.802) (end 45.675 65.223) (width 0.25) (layer "F.Cu") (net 15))
 (segment (start 49.384 56.28) (end 49.384 55.1) (width 0.25) (layer "F.Cu") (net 16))
 (segment (start 48.253802 57.410198) (end 49.384 56.28) (width 0.25) (layer "F.Cu") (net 16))
 (segment (start 48.327802 65.335802) (end 46.424198 65.335802) (width 0.25) (layer "F.Cu") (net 16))
 (segment (start 46.125 65.036604) (end 46.125 57.763792) (width 0.25) (layer "F.Cu") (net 16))
 (segment (start 46.424198 65.335802) (end 46.125 65.036604) (width 0.25) (layer "F.Cu") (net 16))
 (segment (start 46.478594 57.410198) (end 48.253802 57.410198) (width 0.25) (layer "F.Cu") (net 16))
 (segment (start 49.794 66.802) (end 48.327802 65.335802) (width 0.25) (layer "F.Cu") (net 16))
 (segment (start 46.125 57.763792) (end 46.478594 57.410198) (width 0.25) (layer "F.Cu") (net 16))
 (segment (start 34.9 60.533863) (end 34.9 61.7205) (width 0.25) (layer "F.Cu") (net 35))
 (segment (start 35.743863 59.69) (end 34.9 60.533863) (width 0.25) (layer "F.Cu") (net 35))
 (segment (start 34.9 61.7205) (end 36.1715 62.992) (width 0.25) (layer "F.Cu") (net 35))
 (segment (start 36.26 59.69) (end 35.743863 59.69) (width 0.25) (layer "F.Cu") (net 35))
 (segment (start 41.5525 62.992) (end 41.4653 62.992) (width 0.25) (layer "F.Cu") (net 4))
 (segment (start 39.9 61.4267) (end 39.9 58.652) (width 0.25) (layer "F.Cu") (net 4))
 (segment (start 39.9 58.652) (end 40.132 58.42) (width 0.25) (layer "F.Cu") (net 4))
 (segment (start 41.4653 62.992) (end 39.9 61.4267) (width 0.25) (layer "F.Cu") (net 4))
 (segment (start 40.132 58.42) (end 41.21 58.42) (width 0.25) (layer "F.Cu") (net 4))
 (segment (start 34.93 55.82) (end 36.26 57.15) (width 0.25) (layer "F.Cu") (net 33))
 (segment (start 31.75 55.82) (end 34.93 55.82) (width 0.25) (layer "F.Cu") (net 33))
 (segment (start 31.75 61.02) (end 34.35 58.42) (width 0.25) (layer "F.Cu") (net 34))
 (segment (start 34.35 58.42) (end 36.26 58.42) (width 0.25) (layer "F.Cu") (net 34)))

